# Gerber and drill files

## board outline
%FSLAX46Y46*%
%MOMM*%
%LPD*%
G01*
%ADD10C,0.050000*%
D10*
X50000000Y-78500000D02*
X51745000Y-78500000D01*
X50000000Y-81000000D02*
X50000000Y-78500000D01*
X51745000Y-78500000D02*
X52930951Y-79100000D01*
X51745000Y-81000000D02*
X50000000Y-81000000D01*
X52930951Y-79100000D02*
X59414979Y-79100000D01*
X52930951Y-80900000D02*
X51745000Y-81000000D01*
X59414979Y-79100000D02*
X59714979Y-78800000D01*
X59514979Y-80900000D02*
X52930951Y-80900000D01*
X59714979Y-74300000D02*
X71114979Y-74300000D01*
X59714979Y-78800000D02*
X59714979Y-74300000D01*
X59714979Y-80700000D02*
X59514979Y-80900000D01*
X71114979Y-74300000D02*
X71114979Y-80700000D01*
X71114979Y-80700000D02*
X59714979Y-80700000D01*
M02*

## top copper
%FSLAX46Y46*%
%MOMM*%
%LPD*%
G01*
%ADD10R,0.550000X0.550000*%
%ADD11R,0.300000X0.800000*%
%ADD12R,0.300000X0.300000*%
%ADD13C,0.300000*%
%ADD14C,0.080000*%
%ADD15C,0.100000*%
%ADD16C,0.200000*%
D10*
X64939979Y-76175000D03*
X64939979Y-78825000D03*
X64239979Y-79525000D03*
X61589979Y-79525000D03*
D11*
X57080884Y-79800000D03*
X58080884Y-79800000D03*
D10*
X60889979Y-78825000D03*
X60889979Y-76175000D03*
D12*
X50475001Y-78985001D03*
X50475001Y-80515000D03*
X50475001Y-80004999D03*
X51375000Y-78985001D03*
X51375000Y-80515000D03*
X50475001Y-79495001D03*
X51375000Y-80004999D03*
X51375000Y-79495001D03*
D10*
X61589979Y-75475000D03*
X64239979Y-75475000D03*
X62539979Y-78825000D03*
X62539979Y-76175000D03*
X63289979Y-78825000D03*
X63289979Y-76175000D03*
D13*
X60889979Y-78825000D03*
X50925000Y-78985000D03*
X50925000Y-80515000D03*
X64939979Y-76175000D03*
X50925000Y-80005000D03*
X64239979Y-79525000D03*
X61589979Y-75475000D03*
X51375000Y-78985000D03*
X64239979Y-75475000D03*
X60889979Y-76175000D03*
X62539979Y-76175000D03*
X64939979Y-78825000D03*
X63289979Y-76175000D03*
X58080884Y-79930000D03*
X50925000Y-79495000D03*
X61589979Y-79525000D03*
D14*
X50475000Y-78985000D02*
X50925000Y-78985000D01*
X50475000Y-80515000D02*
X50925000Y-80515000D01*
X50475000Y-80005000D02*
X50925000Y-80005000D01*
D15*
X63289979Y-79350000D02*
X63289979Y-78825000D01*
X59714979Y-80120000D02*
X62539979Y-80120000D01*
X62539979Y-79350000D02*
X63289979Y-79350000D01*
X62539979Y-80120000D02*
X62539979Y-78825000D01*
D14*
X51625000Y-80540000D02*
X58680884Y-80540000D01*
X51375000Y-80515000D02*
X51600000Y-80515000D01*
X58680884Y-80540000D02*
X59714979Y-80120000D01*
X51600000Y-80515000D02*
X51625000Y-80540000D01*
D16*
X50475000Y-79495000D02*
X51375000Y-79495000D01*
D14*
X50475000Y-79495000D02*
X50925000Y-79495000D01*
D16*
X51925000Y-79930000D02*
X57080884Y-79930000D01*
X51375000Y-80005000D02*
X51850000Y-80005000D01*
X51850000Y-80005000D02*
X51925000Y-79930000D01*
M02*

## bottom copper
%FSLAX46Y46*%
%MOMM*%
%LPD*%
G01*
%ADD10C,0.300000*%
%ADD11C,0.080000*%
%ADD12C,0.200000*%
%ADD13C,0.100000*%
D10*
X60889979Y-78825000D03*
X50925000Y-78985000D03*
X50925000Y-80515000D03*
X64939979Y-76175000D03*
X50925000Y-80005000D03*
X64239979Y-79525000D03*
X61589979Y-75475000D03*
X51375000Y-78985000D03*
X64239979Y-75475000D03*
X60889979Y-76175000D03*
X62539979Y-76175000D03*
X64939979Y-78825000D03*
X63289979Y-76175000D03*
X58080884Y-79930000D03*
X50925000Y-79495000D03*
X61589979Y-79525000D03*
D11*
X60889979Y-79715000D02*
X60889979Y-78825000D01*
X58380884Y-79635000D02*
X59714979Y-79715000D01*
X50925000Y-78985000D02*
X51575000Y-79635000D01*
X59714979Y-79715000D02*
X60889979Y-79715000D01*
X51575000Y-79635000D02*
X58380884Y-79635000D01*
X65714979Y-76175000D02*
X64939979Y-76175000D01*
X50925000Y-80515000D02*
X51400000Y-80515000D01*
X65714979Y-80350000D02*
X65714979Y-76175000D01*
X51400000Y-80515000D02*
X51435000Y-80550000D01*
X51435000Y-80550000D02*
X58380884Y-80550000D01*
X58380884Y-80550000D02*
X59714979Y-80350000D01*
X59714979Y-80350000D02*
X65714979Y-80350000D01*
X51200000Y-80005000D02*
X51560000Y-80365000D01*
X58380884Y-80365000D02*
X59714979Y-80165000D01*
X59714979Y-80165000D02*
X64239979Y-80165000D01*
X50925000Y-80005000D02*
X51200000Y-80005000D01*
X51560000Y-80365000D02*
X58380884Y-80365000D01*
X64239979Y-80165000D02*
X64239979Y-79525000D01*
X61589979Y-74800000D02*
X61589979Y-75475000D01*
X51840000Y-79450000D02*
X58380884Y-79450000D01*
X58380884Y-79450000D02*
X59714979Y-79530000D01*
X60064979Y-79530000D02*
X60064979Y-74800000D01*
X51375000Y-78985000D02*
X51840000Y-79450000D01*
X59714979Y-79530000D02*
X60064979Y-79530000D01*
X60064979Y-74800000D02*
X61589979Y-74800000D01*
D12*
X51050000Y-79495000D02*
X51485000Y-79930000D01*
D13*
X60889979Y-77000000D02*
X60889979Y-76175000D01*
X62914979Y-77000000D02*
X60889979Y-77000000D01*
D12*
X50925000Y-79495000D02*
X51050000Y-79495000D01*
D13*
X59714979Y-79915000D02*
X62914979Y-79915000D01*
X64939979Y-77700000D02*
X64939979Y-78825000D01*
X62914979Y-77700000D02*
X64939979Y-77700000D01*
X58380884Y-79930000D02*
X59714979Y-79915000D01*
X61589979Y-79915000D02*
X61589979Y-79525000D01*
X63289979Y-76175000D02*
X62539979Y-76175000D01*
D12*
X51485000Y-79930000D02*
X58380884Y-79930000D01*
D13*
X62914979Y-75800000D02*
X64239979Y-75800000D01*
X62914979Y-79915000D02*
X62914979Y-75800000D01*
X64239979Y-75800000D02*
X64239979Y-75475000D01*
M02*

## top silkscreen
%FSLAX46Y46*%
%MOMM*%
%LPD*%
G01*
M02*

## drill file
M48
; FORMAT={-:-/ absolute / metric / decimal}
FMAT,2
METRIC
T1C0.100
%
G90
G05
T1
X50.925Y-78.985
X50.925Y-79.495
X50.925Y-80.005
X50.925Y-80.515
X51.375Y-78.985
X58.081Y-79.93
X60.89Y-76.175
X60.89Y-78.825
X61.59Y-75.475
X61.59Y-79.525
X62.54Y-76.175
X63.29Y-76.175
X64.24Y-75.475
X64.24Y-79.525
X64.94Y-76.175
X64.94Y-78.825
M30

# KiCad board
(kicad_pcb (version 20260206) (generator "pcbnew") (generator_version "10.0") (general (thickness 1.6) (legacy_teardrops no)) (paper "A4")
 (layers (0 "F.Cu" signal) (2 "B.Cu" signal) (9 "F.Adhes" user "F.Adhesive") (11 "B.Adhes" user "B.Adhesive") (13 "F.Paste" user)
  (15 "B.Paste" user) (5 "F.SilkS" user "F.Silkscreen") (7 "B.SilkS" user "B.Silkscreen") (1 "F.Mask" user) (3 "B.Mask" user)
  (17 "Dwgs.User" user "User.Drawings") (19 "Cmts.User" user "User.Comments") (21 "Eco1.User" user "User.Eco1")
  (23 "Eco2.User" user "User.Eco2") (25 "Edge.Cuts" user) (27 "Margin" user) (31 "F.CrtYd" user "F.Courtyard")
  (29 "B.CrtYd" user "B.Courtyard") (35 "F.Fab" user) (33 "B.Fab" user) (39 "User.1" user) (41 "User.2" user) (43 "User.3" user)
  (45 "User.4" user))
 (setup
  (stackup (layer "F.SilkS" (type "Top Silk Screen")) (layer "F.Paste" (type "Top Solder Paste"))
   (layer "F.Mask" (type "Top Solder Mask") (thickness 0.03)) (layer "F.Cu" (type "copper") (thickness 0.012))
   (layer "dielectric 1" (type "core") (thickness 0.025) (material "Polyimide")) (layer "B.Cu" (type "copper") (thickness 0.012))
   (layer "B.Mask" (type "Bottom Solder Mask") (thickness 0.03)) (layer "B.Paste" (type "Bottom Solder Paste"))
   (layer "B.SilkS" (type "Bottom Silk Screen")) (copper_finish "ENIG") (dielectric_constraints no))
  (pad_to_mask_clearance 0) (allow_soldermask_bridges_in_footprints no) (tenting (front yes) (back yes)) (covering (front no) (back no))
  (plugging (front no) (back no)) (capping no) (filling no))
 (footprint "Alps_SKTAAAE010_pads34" (layer "F.Cu") (at 65.314979 77.5 -90)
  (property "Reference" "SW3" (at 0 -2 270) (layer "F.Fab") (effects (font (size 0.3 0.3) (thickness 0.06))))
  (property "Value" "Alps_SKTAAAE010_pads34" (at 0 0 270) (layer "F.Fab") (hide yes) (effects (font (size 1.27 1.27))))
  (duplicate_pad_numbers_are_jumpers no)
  (pad "3" smd rect (at -1.325 0.375 270) (size 0.55 0.55) (layers "F.Cu" "F.Mask") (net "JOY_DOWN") (solder_mask_margin 0.05)
   (thermal_bridge_angle 45))
  (pad "4" smd rect (at 1.325 0.375 270) (size 0.55 0.55) (layers "F.Cu" "F.Mask") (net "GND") (solder_mask_margin 0.05)
   (thermal_bridge_angle 45)))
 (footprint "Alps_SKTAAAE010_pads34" (layer "F.Cu") (at 62.914979 79.9 180)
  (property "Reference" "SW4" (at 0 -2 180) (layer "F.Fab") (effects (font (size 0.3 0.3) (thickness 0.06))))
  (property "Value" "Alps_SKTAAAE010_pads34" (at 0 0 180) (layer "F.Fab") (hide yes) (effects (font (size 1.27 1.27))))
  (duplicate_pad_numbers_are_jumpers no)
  (pad "3" smd rect (at -1.325 0.375 180) (size 0.55 0.55) (layers "F.Cu" "F.Mask") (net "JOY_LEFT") (solder_mask_margin 0.05)
   (thermal_bridge_angle 45))
  (pad "4" smd rect (at 1.325 0.375 180) (size 0.55 0.55) (layers "F.Cu" "F.Mask") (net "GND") (solder_mask_margin 0.05)
   (thermal_bridge_angle 45)))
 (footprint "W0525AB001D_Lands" (layer "F.Cu") (at 57.580884 79.93)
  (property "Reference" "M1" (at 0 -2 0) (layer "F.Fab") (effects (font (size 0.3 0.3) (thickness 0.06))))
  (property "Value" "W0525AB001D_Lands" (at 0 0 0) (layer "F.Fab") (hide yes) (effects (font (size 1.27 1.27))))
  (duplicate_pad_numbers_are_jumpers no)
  (pad "1" smd rect (at -0.5 -0.13) (size 0.3 0.8) (layers "F.Cu" "F.Mask") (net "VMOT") (solder_mask_margin 0.05) (thermal_bridge_angle 45))
  (pad "2" smd rect (at 0.5 -0.13) (size 0.3 0.8) (layers "F.Cu" "F.Mask") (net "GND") (solder_mask_margin 0.05) (thermal_bridge_angle 45)))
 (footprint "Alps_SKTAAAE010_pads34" (layer "F.Cu") (at 60.514979 77.5 90)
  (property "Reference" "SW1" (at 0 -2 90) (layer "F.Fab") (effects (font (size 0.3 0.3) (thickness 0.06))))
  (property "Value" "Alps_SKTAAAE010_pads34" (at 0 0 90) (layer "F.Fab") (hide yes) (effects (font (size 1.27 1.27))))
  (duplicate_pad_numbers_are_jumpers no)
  (pad "3" smd rect (at -1.325 0.375 90) (size 0.55 0.55) (layers "F.Cu" "F.Mask") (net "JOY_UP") (solder_mask_margin 0.05)
   (thermal_bridge_angle 45))
  (pad "4" smd rect (at 1.325 0.375 90) (size 0.55 0.55) (layers "F.Cu" "F.Mask") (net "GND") (solder_mask_margin 0.05)
   (thermal_bridge_angle 45)))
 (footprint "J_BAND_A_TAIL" (layer "F.Cu") (at 50.9 79.75)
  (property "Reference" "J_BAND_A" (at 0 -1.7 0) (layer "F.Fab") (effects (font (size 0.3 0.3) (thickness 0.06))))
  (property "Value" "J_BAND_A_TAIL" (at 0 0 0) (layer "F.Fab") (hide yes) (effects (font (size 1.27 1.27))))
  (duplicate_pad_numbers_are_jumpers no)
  (pad "1" smd rect (at -0.424999 -0.764999) (size 0.3 0.3) (layers "F.Cu" "F.Mask") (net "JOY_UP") (solder_mask_margin 0.05)
   (thermal_bridge_angle 45))
  (pad "2" smd rect (at -0.424999 0.765) (size 0.3 0.3) (layers "F.Cu" "F.Mask") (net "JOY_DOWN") (solder_mask_margin 0.05)
   (thermal_bridge_angle 45))
  (pad "3" smd rect (at -0.424999 0.254999) (size 0.3 0.3) (layers "F.Cu" "F.Mask") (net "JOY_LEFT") (solder_mask_margin 0.05)
   (thermal_bridge_angle 45))
  (pad "4" smd rect (at 0.475 -0.764999) (size 0.3 0.3) (layers "F.Cu" "F.Mask") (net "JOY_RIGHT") (solder_mask_margin 0.05)
   (thermal_bridge_angle 45))
  (pad "5" smd rect (at 0.475 0.765) (size 0.3 0.3) (layers "F.Cu" "F.Mask") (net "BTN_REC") (solder_mask_margin 0.05)
   (thermal_bridge_angle 45))
  (pad "6" smd rect (at -0.424999 -0.254999) (size 0.3 0.3) (layers "F.Cu" "F.Mask") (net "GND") (solder_mask_margin 0.05)
   (thermal_bridge_angle 45))
  (pad "7" smd rect (at 0.475 0.254999) (size 0.3 0.3) (layers "F.Cu" "F.Mask") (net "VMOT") (solder_mask_margin 0.05)
   (thermal_bridge_angle 45))
  (pad "8" smd rect (at 0.475 -0.254999) (size 0.3 0.3) (layers "F.Cu" "F.Mask") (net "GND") (solder_mask_margin 0.05)
   (thermal_bridge_angle 45)))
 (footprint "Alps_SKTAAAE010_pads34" (layer "F.Cu") (at 62.914979 75.1)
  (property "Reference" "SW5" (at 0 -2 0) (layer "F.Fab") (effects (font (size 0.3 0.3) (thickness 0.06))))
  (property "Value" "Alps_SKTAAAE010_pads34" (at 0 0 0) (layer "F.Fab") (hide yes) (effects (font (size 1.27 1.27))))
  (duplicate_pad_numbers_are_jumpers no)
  (pad "3" smd rect (at -1.325 0.375) (size 0.55 0.55) (layers "F.Cu" "F.Mask") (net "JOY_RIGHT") (solder_mask_margin 0.05)
   (thermal_bridge_angle 45))
  (pad "4" smd rect (at 1.325 0.375) (size 0.55 0.55) (layers "F.Cu" "F.Mask") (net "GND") (solder_mask_margin 0.05)
   (thermal_bridge_angle 45)))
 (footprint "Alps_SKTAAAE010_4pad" (layer "F.Cu") (at 62.914979 77.5 90)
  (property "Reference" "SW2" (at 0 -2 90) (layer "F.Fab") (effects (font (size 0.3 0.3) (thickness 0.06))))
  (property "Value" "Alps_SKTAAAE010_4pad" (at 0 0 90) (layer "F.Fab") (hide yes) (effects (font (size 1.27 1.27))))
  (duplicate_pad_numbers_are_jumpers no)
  (pad "1" smd rect (at -1.325 -0.375 90) (size 0.55 0.55) (layers "F.Cu" "F.Mask") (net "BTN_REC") (solder_mask_margin 0.05)
   (thermal_bridge_angle 45))
  (pad "2" smd rect (at 1.325 -0.375 90) (size 0.55 0.55) (layers "F.Cu" "F.Mask") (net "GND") (solder_mask_margin 0.05)
   (thermal_bridge_angle 45))
  (pad "3" smd rect (at -1.325 0.375 90) (size 0.55 0.55) (layers "F.Cu" "F.Mask") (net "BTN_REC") (solder_mask_margin 0.05)
   (thermal_bridge_angle 45))
  (pad "4" smd rect (at 1.325 0.375 90) (size 0.55 0.55) (layers "F.Cu" "F.Mask") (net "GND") (solder_mask_margin 0.05)
   (thermal_bridge_angle 45)))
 (gr_line (start 50 78.5) (end 51.745 78.5) (stroke (width 0.05) (type default)) (layer "Edge.Cuts"))
 (gr_line (start 50 81) (end 50 78.5) (stroke (width 0.05) (type default)) (layer "Edge.Cuts"))
 (gr_line (start 51.745 78.5) (end 52.930951 79.1) (stroke (width 0.05) (type default)) (layer "Edge.Cuts"))
 (gr_line (start 51.745 81) (end 50 81) (stroke (width 0.05) (type default)) (layer "Edge.Cuts"))
 (gr_line (start 52.930951 79.1) (end 59.414979 79.1) (stroke (width 0.05) (type default)) (layer "Edge.Cuts"))
 (gr_line (start 52.930951 80.9) (end 51.745 81) (stroke (width 0.05) (type default)) (layer "Edge.Cuts"))
 (gr_line (start 59.414979 79.1) (end 59.714979 78.8) (stroke (width 0.05) (type default)) (layer "Edge.Cuts"))
 (gr_line (start 59.514979 80.9) (end 52.930951 80.9) (stroke (width 0.05) (type default)) (layer "Edge.Cuts"))
 (gr_line (start 59.714979 74.3) (end 71.114979 74.3) (stroke (width 0.05) (type default)) (layer "Edge.Cuts"))
 (gr_line (start 59.714979 78.8) (end 59.714979 74.3) (stroke (width 0.05) (type default)) (layer "Edge.Cuts"))
 (gr_line (start 59.714979 80.7) (end 59.514979 80.9) (stroke (width 0.05) (type default)) (layer "Edge.Cuts"))
 (gr_line (start 71.114979 74.3) (end 71.114979 80.7) (stroke (width 0.05) (type default)) (layer "Edge.Cuts"))
 (gr_line (start 71.114979 80.7) (end 59.714979 80.7) (stroke (width 0.05) (type default)) (layer "Edge.Cuts"))
 (segment (start 50.475 78.985) (end 50.925 78.985) (width 0.08) (layer "F.Cu") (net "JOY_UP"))
 (via (at 60.889979 78.825) (size 0.3) (drill 0.1) (layers "F.Cu" "B.Cu") (tenting (front yes) (back yes)) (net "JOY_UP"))
 (via (at 50.925 78.985) (size 0.3) (drill 0.1) (layers "F.Cu" "B.Cu") (tenting (front yes) (back yes)) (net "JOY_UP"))
 (segment (start 60.889979 79.715) (end 60.889979 78.825) (width 0.08) (layer "B.Cu") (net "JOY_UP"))
 (segment (start 58.380884 79.635) (end 59.714979 79.715) (width 0.08) (layer "B.Cu") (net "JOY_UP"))
 (segment (start 50.925 78.985) (end 51.575 79.635) (width 0.08) (layer "B.Cu") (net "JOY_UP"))
 (segment (start 59.714979 79.715) (end 60.889979 79.715) (width 0.08) (layer "B.Cu") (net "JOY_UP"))
 (segment (start 51.575 79.635) (end 58.380884 79.635) (width 0.08) (layer "B.Cu") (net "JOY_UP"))
 (segment (start 50.475 80.515) (end 50.925 80.515) (width 0.08) (layer "F.Cu") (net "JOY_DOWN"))
 (via (at 50.925 80.515) (size 0.3) (drill 0.1) (layers "F.Cu" "B.Cu") (tenting (front yes) (back yes)) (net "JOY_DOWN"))
 (via (at 64.939979 76.175) (size 0.3) (drill 0.1) (layers "F.Cu" "B.Cu") (tenting (front yes) (back yes)) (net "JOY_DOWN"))
 (segment (start 65.714979 76.175) (end 64.939979 76.175) (width 0.08) (layer "B.Cu") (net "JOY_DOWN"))
 (segment (start 50.925 80.515) (end 51.4 80.515) (width 0.08) (layer "B.Cu") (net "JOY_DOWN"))
 (segment (start 65.714979 80.35) (end 65.714979 76.175) (width 0.08) (layer "B.Cu") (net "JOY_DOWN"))
 (segment (start 51.4 80.515) (end 51.435 80.55) (width 0.08) (layer "B.Cu") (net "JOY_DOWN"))
 (segment (start 51.435 80.55) (end 58.380884 80.55) (width 0.08) (layer "B.Cu") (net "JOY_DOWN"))
 (segment (start 58.380884 80.55) (end 59.714979 80.35) (width 0.08) (layer "B.Cu") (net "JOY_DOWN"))
 (segment (start 59.714979 80.35) (end 65.714979 80.35) (width 0.08) (layer "B.Cu") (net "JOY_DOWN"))
 (segment (start 50.475 80.005) (end 50.925 80.005) (width 0.08) (layer "F.Cu") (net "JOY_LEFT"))
 (via (at 50.925 80.005) (size 0.3) (drill 0.1) (layers "F.Cu" "B.Cu") (tenting (front yes) (back yes)) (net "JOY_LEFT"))
 (via (at 64.239979 79.525) (size 0.3) (drill 0.1) (layers "F.Cu" "B.Cu") (tenting (front yes) (back yes)) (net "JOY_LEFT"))
 (segment (start 51.2 80.005) (end 51.56 80.365) (width 0.08) (layer "B.Cu") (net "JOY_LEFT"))
 (segment (start 58.380884 80.365) (end 59.714979 80.165) (width 0.08) (layer "B.Cu") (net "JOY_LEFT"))
 (segment (start 59.714979 80.165) (end 64.239979 80.165) (width 0.08) (layer "B.Cu") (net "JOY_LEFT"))
 (segment (start 50.925 80.005) (end 51.2 80.005) (width 0.08) (layer "B.Cu") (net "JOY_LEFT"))
 (segment (start 51.56 80.365) (end 58.380884 80.365) (width 0.08) (layer "B.Cu") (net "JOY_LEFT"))
 (segment (start 64.239979 80.165) (end 64.239979 79.525) (width 0.08) (layer "B.Cu") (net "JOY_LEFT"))
 (via (at 61.589979 75.475) (size 0.3) (drill 0.1) (layers "F.Cu" "B.Cu") (tenting (front yes) (back yes)) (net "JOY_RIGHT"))
 (via (at 51.375 78.985) (size 0.3) (drill 0.1) (layers "F.Cu" "B.Cu") (tenting (front yes) (back yes)) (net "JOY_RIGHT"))
 (segment (start 61.589979 74.8) (end 61.589979 75.475) (width 0.08) (layer "B.Cu") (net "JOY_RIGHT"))
 (segment (start 51.84 79.45) (end 58.380884 79.45) (width 0.08) (layer "B.Cu") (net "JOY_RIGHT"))
 (segment (start 58.380884 79.45) (end 59.714979 79.53) (width 0.08) (layer "B.Cu") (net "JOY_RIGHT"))
 (segment (start 60.064979 79.53) (end 60.064979 74.8) (width 0.08) (layer "B.Cu") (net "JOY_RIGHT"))
 (segment (start 51.375 78.985) (end 51.84 79.45) (width 0.08) (layer "B.Cu") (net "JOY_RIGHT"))
 (segment (start 59.714979 79.53) (end 60.064979 79.53) (width 0.08) (layer "B.Cu") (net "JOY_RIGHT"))
 (segment (start 60.064979 74.8) (end 61.589979 74.8) (width 0.08) (layer "B.Cu") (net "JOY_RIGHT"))
 (segment (start 63.289979 79.35) (end 63.289979 78.825) (width 0.1) (layer "F.Cu") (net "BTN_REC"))
 (segment (start 59.714979 80.12) (end 62.539979 80.12) (width 0.1) (layer "F.Cu") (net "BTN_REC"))
 (segment (start 62.539979 79.35) (end 63.289979 79.35) (width 0.1) (layer "F.Cu") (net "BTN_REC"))
 (segment (start 62.539979 80.12) (end 62.539979 78.825) (width 0.1) (layer "F.Cu") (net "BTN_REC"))
 (segment (start 51.625 80.54) (end 58.680884 80.54) (width 0.08) (layer "F.Cu") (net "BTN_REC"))
 (segment (start 51.375 80.515) (end 51.6 80.515) (width 0.08) (layer "F.Cu") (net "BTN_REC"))
 (segment (start 58.680884 80.54) (end 59.714979 80.12) (width 0.08) (layer "F.Cu") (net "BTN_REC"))
 (segment (start 51.6 80.515) (end 51.625 80.54) (width 0.08) (layer "F.Cu") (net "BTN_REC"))
 (segment (start 50.475 79.495) (end 51.375 79.495) (width 0.2) (layer "F.Cu") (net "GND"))
 (segment (start 50.475 79.495) (end 50.925 79.495) (width 0.08) (layer "F.Cu") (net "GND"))
 (via (at 64.239979 75.475) (size 0.3) (drill 0.1) (layers "F.Cu" "B.Cu") (tenting (front yes) (back yes)) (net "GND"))
 (via (at 60.889979 76.175) (size 0.3) (drill 0.1) (layers "F.Cu" "B.Cu") (tenting (front yes) (back yes)) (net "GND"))
 (via (at 62.539979 76.175) (size 0.3) (drill 0.1) (layers "F.Cu" "B.Cu") (tenting (front yes) (back yes)) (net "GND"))
 (via (at 64.939979 78.825) (size 0.3) (drill 0.1) (layers "F.Cu" "B.Cu") (tenting (front yes) (back yes)) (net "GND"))
 (via (at 63.289979 76.175) (size 0.3) (drill 0.1) (layers "F.Cu" "B.Cu") (tenting (front yes) (back yes)) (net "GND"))
 (via (at 58.080884 79.93) (size 0.3) (drill 0.1) (layers "F.Cu" "B.Cu") (tenting (front yes) (back yes)) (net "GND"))
 (via (at 50.925 79.495) (size 0.3) (drill 0.1) (layers "F.Cu" "B.Cu") (tenting (front yes) (back yes)) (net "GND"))
 (via (at 61.589979 79.525) (size 0.3) (drill 0.1) (layers "F.Cu" "B.Cu") (tenting (front yes) (back yes)) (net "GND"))
 (segment (start 51.05 79.495) (end 51.485 79.93) (width 0.2) (layer "B.Cu") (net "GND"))
 (segment (start 60.889979 77) (end 60.889979 76.175) (width 0.1) (layer "B.Cu") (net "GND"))
 (segment (start 62.914979 77) (end 60.889979 77) (width 0.1) (layer "B.Cu") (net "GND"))
 (segment (start 50.925 79.495) (end 51.05 79.495) (width 0.2) (layer "B.Cu") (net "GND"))
 (segment (start 59.714979 79.915) (end 62.914979 79.915) (width 0.1) (layer "B.Cu") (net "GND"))
 (segment (start 64.939979 77.7) (end 64.939979 78.825) (width 0.1) (layer "B.Cu") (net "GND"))
 (segment (start 62.914979 77.7) (end 64.939979 77.7) (width 0.1) (layer "B.Cu") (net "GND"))
 (segment (start 58.380884 79.93) (end 59.714979 79.915) (width 0.1) (layer "B.Cu") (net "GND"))
 (segment (start 61.589979 79.915) (end 61.589979 79.525) (width 0.1) (layer "B.Cu") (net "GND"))
 (segment (start 63.289979 76.175) (end 62.539979 76.175) (width 0.1) (layer "B.Cu") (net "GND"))
 (segment (start 51.485 79.93) (end 58.380884 79.93) (width 0.2) (layer "B.Cu") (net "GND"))
 (segment (start 62.914979 75.8) (end 64.239979 75.8) (width 0.1) (layer "B.Cu") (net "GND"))
 (segment (start 62.914979 79.915) (end 62.914979 75.8) (width 0.1) (layer "B.Cu") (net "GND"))
 (segment (start 64.239979 75.8) (end 64.239979 75.475) (width 0.1) (layer "B.Cu") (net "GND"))
 (segment (start 51.925 79.93) (end 57.080884 79.93) (width 0.2) (layer "F.Cu") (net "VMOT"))
 (segment (start 51.375 80.005) (end 51.85 80.005) (width 0.2) (layer "F.Cu") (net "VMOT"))
 (segment (start 51.85 80.005) (end 51.925 79.93) (width 0.2) (layer "F.Cu") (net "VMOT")))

